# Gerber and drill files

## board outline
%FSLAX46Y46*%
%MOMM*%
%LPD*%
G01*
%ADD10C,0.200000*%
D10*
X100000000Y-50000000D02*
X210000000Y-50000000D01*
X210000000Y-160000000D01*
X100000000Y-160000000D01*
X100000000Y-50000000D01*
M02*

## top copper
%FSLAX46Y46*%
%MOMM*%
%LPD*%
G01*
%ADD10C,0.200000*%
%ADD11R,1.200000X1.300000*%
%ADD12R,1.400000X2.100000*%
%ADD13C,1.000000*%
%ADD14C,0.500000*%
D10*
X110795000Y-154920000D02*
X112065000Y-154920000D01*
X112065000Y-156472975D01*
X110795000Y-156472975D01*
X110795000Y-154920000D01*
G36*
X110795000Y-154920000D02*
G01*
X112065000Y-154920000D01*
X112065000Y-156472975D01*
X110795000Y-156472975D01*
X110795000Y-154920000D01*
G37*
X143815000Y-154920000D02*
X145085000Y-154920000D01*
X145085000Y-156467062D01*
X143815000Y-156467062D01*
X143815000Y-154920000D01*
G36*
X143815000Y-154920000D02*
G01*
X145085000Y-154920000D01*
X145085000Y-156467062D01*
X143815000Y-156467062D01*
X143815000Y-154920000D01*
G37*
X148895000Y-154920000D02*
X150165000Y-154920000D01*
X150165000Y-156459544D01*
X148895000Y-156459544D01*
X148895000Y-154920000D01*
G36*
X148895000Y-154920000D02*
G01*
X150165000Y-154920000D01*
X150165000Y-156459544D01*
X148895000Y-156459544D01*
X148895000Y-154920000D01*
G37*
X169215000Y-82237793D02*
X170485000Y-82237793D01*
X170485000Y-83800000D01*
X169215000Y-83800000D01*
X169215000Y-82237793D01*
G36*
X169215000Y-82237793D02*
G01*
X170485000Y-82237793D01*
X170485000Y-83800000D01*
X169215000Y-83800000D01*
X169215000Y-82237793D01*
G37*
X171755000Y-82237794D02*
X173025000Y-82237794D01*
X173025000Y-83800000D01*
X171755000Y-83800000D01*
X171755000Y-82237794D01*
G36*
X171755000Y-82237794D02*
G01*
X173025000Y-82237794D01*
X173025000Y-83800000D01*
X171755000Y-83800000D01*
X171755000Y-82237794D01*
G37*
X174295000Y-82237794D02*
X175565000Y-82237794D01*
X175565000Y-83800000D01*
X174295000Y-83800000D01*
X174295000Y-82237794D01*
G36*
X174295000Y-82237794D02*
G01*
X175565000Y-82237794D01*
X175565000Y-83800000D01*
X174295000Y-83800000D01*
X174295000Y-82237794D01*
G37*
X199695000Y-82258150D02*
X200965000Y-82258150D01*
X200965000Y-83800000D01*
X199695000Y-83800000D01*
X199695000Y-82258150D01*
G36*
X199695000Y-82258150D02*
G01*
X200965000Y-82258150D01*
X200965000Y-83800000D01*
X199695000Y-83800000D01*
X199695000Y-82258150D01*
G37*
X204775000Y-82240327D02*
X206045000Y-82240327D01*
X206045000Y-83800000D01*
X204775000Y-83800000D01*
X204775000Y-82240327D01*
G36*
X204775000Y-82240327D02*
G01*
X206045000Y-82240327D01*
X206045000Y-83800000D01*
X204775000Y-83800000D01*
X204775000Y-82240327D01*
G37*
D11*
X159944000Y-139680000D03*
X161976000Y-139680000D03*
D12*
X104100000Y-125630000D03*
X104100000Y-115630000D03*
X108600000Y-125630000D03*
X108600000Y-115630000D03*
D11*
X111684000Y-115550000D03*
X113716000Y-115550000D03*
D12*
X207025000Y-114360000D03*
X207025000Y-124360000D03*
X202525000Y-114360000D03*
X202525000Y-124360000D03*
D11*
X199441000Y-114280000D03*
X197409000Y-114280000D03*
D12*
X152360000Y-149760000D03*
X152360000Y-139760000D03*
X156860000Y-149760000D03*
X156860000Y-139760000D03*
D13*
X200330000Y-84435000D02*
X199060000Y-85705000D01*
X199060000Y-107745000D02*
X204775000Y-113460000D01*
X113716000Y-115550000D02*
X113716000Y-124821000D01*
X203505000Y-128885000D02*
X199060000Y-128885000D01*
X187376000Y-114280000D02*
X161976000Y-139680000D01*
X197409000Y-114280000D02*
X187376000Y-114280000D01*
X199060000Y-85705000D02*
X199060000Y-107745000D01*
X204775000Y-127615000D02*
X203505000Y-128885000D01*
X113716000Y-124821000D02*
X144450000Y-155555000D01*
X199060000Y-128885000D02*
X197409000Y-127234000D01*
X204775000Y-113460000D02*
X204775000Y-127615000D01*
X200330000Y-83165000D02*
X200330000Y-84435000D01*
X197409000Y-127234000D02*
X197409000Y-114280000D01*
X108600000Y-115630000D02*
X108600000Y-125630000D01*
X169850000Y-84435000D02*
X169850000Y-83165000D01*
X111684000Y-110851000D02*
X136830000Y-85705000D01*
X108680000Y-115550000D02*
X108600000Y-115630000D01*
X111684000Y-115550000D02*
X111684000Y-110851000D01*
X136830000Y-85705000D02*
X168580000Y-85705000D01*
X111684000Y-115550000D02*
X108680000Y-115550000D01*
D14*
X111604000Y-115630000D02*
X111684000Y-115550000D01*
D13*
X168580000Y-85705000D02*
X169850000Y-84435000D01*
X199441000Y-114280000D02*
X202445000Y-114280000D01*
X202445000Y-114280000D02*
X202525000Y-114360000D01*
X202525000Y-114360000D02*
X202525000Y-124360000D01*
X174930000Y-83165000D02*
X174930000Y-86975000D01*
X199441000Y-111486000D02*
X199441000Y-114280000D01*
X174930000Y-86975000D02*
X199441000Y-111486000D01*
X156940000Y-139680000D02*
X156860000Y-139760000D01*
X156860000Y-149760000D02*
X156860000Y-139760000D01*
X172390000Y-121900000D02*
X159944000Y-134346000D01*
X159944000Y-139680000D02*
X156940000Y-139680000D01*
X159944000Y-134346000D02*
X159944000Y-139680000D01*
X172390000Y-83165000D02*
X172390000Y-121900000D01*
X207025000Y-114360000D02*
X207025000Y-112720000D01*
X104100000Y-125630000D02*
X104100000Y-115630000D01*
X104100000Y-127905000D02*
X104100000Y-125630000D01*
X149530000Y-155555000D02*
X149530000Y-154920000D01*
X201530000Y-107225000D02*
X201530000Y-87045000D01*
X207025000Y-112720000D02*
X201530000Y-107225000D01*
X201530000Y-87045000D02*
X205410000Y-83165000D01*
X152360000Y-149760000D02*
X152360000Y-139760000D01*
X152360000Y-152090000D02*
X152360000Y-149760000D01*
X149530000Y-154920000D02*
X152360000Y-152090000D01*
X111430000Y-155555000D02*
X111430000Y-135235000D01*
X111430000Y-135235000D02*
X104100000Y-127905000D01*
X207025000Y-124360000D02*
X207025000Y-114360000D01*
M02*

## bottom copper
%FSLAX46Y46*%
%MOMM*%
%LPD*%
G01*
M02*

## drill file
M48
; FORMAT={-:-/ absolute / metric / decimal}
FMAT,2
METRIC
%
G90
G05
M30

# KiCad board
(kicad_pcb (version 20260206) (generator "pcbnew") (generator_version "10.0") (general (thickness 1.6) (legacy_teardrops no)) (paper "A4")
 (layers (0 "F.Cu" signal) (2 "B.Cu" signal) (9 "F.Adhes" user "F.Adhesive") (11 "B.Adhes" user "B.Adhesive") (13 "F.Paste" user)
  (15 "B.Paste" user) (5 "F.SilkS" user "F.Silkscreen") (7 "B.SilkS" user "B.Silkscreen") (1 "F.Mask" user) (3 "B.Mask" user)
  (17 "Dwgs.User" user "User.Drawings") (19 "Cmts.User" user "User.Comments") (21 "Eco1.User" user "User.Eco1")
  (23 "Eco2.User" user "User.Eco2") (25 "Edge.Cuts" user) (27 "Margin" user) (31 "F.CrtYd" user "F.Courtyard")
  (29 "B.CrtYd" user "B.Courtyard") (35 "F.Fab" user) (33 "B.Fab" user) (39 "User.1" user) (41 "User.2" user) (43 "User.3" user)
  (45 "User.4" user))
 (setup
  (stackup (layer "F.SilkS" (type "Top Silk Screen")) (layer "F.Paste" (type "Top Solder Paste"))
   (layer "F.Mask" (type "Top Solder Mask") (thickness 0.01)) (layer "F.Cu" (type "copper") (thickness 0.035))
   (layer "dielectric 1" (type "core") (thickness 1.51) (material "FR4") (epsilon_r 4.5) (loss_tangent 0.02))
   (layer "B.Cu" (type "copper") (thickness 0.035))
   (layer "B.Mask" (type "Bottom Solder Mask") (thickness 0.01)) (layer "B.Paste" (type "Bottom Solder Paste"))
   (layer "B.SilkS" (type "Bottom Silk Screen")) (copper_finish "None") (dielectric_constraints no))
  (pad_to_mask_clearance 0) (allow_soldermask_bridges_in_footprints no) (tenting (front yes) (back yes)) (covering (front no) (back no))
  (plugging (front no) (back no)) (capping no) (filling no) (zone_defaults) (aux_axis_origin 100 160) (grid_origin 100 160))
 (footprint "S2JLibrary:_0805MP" (layer "F.Cu") (at 160.96 139.68)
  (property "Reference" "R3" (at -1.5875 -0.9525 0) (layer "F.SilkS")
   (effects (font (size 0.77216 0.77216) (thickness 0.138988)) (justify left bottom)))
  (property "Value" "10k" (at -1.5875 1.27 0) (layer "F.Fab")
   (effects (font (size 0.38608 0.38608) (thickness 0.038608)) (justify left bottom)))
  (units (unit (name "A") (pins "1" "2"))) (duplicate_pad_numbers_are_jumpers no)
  (pad "1" smd rect (at -1.016 0) (size 1.2 1.3) (layers "F.Cu" "F.Mask" "F.Paste") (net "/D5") (solder_mask_margin 0.1016))
  (pad "2" smd rect (at 1.016 0) (size 1.2 1.3) (layers "F.Cu" "F.Mask" "F.Paste") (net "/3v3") (solder_mask_margin 0.1016)))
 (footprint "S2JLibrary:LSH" (layer "F.Cu") (at 106.35 120.63 90)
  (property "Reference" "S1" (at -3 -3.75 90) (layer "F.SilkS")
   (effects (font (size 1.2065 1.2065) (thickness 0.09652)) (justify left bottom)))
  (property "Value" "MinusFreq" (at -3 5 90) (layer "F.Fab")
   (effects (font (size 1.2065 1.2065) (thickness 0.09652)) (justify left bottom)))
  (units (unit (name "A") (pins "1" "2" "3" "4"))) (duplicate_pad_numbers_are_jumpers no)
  (pad "1" smd rect (at -5 -2.25 90) (size 2.1 1.4) (layers "F.Cu" "F.Mask" "F.Paste") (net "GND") (solder_mask_margin 0.1016))
  (pad "2" smd rect (at 5 -2.25 90) (size 2.1 1.4) (layers "F.Cu" "F.Mask" "F.Paste") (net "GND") (solder_mask_margin 0.1016))
  (pad "3" smd rect (at -5 2.25 90) (size 2.1 1.4) (layers "F.Cu" "F.Mask" "F.Paste") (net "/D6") (solder_mask_margin 0.1016))
  (pad "4" smd rect (at 5 2.25 90) (size 2.1 1.4) (layers "F.Cu" "F.Mask" "F.Paste") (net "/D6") (solder_mask_margin 0.1016)))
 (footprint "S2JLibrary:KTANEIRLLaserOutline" (layer "F.Cu") (at 100 160)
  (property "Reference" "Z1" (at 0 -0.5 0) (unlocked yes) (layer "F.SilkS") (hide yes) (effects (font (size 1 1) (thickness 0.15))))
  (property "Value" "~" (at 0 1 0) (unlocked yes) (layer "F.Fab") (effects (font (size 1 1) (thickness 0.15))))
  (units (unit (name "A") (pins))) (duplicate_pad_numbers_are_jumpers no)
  (pad "" smd circle (at 5 -105 180) (size 5.5 5.5) (layers "F.SilkS") (solder_mask_margin 0.1016) (clearance 1))
  (pad "" smd circle (at 5 -55 180) (size 5.5 5.5) (layers "F.SilkS") (solder_mask_margin 0.1016) (clearance 1))
  (pad "" smd circle (at 5 -5 180) (size 5.5 5.5) (layers "F.SilkS") (solder_mask_margin 0.1016) (clearance 1))
  (pad "" smd circle (at 11.43 -2.54 90) (size 1.6764 1.6764) (layers "F.SilkS") (solder_mask_margin 0.1016))
  (pad "" smd circle (at 13.97 -2.54 90) (size 1.6764 1.6764) (layers "F.SilkS") (solder_mask_margin 0.1016))
  (pad "" smd circle (at 16.51 -2.54 90) (size 1.6764 1.6764) (layers "F.SilkS") (solder_mask_margin 0.1016))
  (pad "" smd circle (at 19.05 -2.54 90) (size 1.6764 1.6764) (layers "F.SilkS") (solder_mask_margin 0.1016))
  (pad "" smd circle (at 21.59 -2.54 90) (size 1.6764 1.6764) (layers "F.SilkS") (solder_mask_margin 0.1016))
  (pad "" smd circle (at 24.13 -2.54 90) (size 1.6764 1.6764) (layers "F.SilkS") (solder_mask_margin 0.1016))
  (pad "" smd circle (at 26.67 -2.54 90) (size 1.6764 1.6764) (layers "F.SilkS") (solder_mask_margin 0.1016))
  (pad "" smd circle (at 29.21 -2.54 90) (size 1.6764 1.6764) (layers "F.SilkS") (solder_mask_margin 0.1016))
  (pad "" smd circle (at 31.75 -2.54 90) (size 1.6764 1.6764) (layers "F.SilkS") (solder_mask_margin 0.1016))
  (pad "" smd circle (at 34.29 -2.54 90) (size 1.6764 1.6764) (layers "F.SilkS") (solder_mask_margin 0.1016))
  (pad "" smd circle (at 36.83 -2.54 90) (size 1.6764 1.6764) (layers "F.SilkS") (solder_mask_margin 0.1016))
  (pad "" smd circle (at 39.37 -2.54 90) (size 1.6764 1.6764) (layers "F.SilkS") (solder_mask_margin 0.1016))
  (pad "" smd circle (at 41.91 -2.54 90) (size 1.6764 1.6764) (layers "F.SilkS") (solder_mask_margin 0.1016))
  (pad "" smd circle (at 44.45 -2.54 90) (size 1.6764 1.6764) (layers "F.SilkS") (solder_mask_margin 0.1016))
  (pad "" smd circle (at 46.99 -2.54 90) (size 1.6764 1.6764) (layers "F.SilkS") (solder_mask_margin 0.1016))
  (pad "" smd circle (at 49.53 -2.54 90) (size 1.6764 1.6764) (layers "F.SilkS") (solder_mask_margin 0.1016))
  (pad "" smd circle (at 55 -105 180) (size 5.5 5.5) (layers "F.SilkS") (solder_mask_margin 0.1016) (clearance 1))
  (pad "" smd circle (at 55 -55 180) (size 5.5 5.5) (layers "F.SilkS") (solder_mask_margin 0.1016) (clearance 1))
  (pad "" smd circle (at 55 -5 180) (size 5.5 5.5) (layers "F.SilkS") (solder_mask_margin 0.1016) (clearance 1))
  (pad "" smd circle (at 67.31 -81.28 90) (size 1.6764 1.6764) (layers "F.SilkS") (solder_mask_margin 0.1016))
  (pad "" smd circle (at 67.31 -78.74 90) (size 1.6764 1.6764) (layers "F.SilkS") (solder_mask_margin 0.1016))
  (pad "" smd circle (at 69.85 -81.28 90) (size 1.6764 1.6764) (layers "F.SilkS") (solder_mask_margin 0.1016))
  (pad "" smd circle (at 69.85 -78.74 90) (size 1.6764 1.6764) (layers "F.SilkS") (solder_mask_margin 0.1016))
  (pad "" smd circle (at 72.39 -81.28 90) (size 1.6764 1.6764) (layers "F.SilkS") (solder_mask_margin 0.1016))
  (pad "" smd circle (at 72.39 -78.74 90) (size 1.6764 1.6764) (layers "F.SilkS") (solder_mask_margin 0.1016))
  (pad "" smd circle (at 74.93 -81.28 90) (size 1.6764 1.6764) (layers "F.SilkS") (solder_mask_margin 0.1016))
  (pad "" smd circle (at 74.93 -78.74 90) (size 1.6764 1.6764) (layers "F.SilkS") (solder_mask_margin 0.1016))
  (pad "" smd circle (at 77.47 -81.28 90) (size 1.6764 1.6764) (layers "F.SilkS") (solder_mask_margin 0.1016))
  (pad "" smd circle (at 77.47 -78.74 90) (size 1.6764 1.6764) (layers "F.SilkS") (solder_mask_margin 0.1016))
  (pad "" smd circle (at 80.01 -81.28 90) (size 1.6764 1.6764) (layers "F.SilkS") (solder_mask_margin 0.1016))
  (pad "" smd circle (at 80.01 -78.74 90) (size 1.6764 1.6764) (layers "F.SilkS") (solder_mask_margin 0.1016))
  (pad "" smd circle (at 82.55 -81.28 90) (size 1.6764 1.6764) (layers "F.SilkS") (solder_mask_margin 0.1016))
  (pad "" smd circle (at 82.55 -78.74 90) (size 1.6764 1.6764) (layers "F.SilkS") (solder_mask_margin 0.1016))
  (pad "" smd circle (at 85.09 -81.28 90) (size 1.6764 1.6764) (layers "F.SilkS") (solder_mask_margin 0.1016))
  (pad "" smd circle (at 85.09 -78.74 90) (size 1.6764 1.6764) (layers "F.SilkS") (solder_mask_margin 0.1016))
  (pad "" smd circle (at 87.63 -81.28 90) (size 1.6764 1.6764) (layers "F.SilkS") (solder_mask_margin 0.1016))
  (pad "" smd circle (at 87.63 -78.74 90) (size 1.6764 1.6764) (layers "F.SilkS") (solder_mask_margin 0.1016))
  (pad "" smd circle (at 90.17 -81.28 90) (size 1.6764 1.6764) (layers "F.SilkS") (solder_mask_margin 0.1016))
  (pad "" smd circle (at 90.17 -78.74 90) (size 1.6764 1.6764) (layers "F.SilkS") (solder_mask_margin 0.1016))
  (pad "" smd circle (at 92.71 -81.28 90) (size 1.6764 1.6764) (layers "F.SilkS") (solder_mask_margin 0.1016))
  (pad "" smd circle (at 92.71 -78.74 90) (size 1.6764 1.6764) (layers "F.SilkS") (solder_mask_margin 0.1016))
  (pad "" smd circle (at 95.25 -81.28 90) (size 1.6764 1.6764) (layers "F.SilkS") (solder_mask_margin 0.1016))
  (pad "" smd circle (at 95.25 -78.74 90) (size 1.6764 1.6764) (layers "F.SilkS") (solder_mask_margin 0.1016))
  (pad "" smd circle (at 97.79 -81.28 90) (size 1.6764 1.6764) (layers "F.SilkS") (solder_mask_margin 0.1016))
  (pad "" smd circle (at 97.79 -78.74 90) (size 1.6764 1.6764) (layers "F.SilkS") (solder_mask_margin 0.1016))
  (pad "" smd circle (at 100.33 -81.28 90) (size 1.6764 1.6764) (layers "F.SilkS") (solder_mask_margin 0.1016))
  (pad "" smd circle (at 100.33 -78.74 90) (size 1.6764 1.6764) (layers "F.SilkS") (solder_mask_margin 0.1016))
  (pad "" smd circle (at 102.87 -81.28 90) (size 1.6764 1.6764) (layers "F.SilkS") (solder_mask_margin 0.1016))
  (pad "" smd circle (at 102.87 -78.74 90) (size 1.6764 1.6764) (layers "F.SilkS") (solder_mask_margin 0.1016))
  (pad "" smd circle (at 105 -55 180) (size 5.5 5.5) (layers "F.SilkS") (solder_mask_margin 0.1016) (clearance 1))
  (pad "" smd circle (at 105 -5 180) (size 5.5 5.5) (layers "F.SilkS") (solder_mask_margin 0.1016) (clearance 1))
  (pad "" smd circle (at 105.41 -81.28 90) (size 1.6764 1.6764) (layers "F.SilkS") (solder_mask_margin 0.1016))
  (pad "" smd circle (at 105.41 -78.74 90) (size 1.6764 1.6764) (layers "F.SilkS") (solder_mask_margin 0.1016)))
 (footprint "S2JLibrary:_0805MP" (layer "F.Cu") (at 112.7 115.55)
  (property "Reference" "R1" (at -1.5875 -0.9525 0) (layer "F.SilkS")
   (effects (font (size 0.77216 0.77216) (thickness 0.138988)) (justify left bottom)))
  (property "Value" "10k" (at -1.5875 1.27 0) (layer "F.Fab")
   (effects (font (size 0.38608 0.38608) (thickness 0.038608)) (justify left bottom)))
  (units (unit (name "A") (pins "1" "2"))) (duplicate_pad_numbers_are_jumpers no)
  (pad "1" smd rect (at -1.016 0) (size 1.2 1.3) (layers "F.Cu" "F.Mask" "F.Paste") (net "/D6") (solder_mask_margin 0.1016))
  (pad "2" smd rect (at 1.016 0) (size 1.2 1.3) (layers "F.Cu" "F.Mask" "F.Paste") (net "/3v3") (solder_mask_margin 0.1016)))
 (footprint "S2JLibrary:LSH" (layer "F.Cu") (at 204.775 119.36 -90)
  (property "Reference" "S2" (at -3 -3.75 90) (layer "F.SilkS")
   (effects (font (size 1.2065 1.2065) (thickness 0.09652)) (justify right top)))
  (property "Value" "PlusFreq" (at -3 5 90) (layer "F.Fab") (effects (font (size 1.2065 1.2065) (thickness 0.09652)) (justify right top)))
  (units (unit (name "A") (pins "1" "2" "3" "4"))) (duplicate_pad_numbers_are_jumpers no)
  (pad "1" smd rect (at -5 -2.25 270) (size 2.1 1.4) (layers "F.Cu" "F.Mask" "F.Paste") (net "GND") (solder_mask_margin 0.1016))
  (pad "2" smd rect (at 5 -2.25 270) (size 2.1 1.4) (layers "F.Cu" "F.Mask" "F.Paste") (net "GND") (solder_mask_margin 0.1016))
  (pad "3" smd rect (at -5 2.25 270) (size 2.1 1.4) (layers "F.Cu" "F.Mask" "F.Paste") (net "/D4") (solder_mask_margin 0.1016))
  (pad "4" smd rect (at 5 2.25 270) (size 2.1 1.4) (layers "F.Cu" "F.Mask" "F.Paste") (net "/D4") (solder_mask_margin 0.1016)))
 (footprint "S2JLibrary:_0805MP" (layer "F.Cu") (at 198.425 114.28 180)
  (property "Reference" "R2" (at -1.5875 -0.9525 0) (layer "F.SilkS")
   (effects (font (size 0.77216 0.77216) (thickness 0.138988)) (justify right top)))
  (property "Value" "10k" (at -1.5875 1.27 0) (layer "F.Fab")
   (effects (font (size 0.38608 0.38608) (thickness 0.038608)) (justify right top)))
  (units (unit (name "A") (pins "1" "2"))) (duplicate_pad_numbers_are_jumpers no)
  (pad "1" smd rect (at -1.016 0 180) (size 1.2 1.3) (layers "F.Cu" "F.Mask" "F.Paste") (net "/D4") (solder_mask_margin 0.1016))
  (pad "2" smd rect (at 1.016 0 180) (size 1.2 1.3) (layers "F.Cu" "F.Mask" "F.Paste") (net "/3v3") (solder_mask_margin 0.1016)))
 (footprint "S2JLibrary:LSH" (layer "F.Cu") (at 154.61 144.76 90)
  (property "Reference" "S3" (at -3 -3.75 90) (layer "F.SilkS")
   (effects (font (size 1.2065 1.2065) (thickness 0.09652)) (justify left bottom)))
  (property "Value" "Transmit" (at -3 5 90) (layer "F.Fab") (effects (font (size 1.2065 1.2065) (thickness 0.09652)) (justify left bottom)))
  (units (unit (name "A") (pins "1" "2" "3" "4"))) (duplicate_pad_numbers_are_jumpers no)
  (pad "1" smd rect (at -5 -2.25 90) (size 2.1 1.4) (layers "F.Cu" "F.Mask" "F.Paste") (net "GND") (solder_mask_margin 0.1016))
  (pad "2" smd rect (at 5 -2.25 90) (size 2.1 1.4) (layers "F.Cu" "F.Mask" "F.Paste") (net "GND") (solder_mask_margin 0.1016))
  (pad "3" smd rect (at -5 2.25 90) (size 2.1 1.4) (layers "F.Cu" "F.Mask" "F.Paste") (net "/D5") (solder_mask_margin 0.1016))
  (pad "4" smd rect (at 5 2.25 90) (size 2.1 1.4) (layers "F.Cu" "F.Mask" "F.Paste") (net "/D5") (solder_mask_margin 0.1016)))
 (gr_rect (start 110.795 154.92) (end 112.065 156.472975) (stroke (width 0.2) (type solid)) (fill yes) (layers "F.Cu" "F.Mask") (net "GND"))
 (gr_rect (start 143.815 154.92) (end 145.085 156.467062) (stroke (width 0.2) (type solid)) (fill yes) (layers "F.Cu" "F.Mask") (net "/3v3"))
 (gr_rect (start 148.895 154.92) (end 150.165 156.459544) (stroke (width 0.2) (type solid)) (fill yes) (layers "F.Cu" "F.Mask") (net "GND"))
 (gr_rect (start 169.215 82.237793) (end 170.485 83.8) (stroke (width 0.2) (type solid)) (fill yes) (layers "F.Cu" "F.Mask") (net "/D6"))
 (gr_rect (start 171.755 82.237794) (end 173.025 83.8) (stroke (width 0.2) (type solid)) (fill yes) (layers "F.Cu" "F.Mask") (net "/D5"))
 (gr_rect (start 174.295 82.237794) (end 175.565 83.8) (stroke (width 0.2) (type solid)) (fill yes) (layers "F.Cu" "F.Mask") (net "/D4"))
 (gr_rect (start 199.695 82.25815) (end 200.965 83.8) (stroke (width 0.2) (type solid)) (fill yes) (layers "F.Cu" "F.Mask") (net "/3v3"))
 (gr_rect (start 204.775 82.240327) (end 206.045 83.8) (stroke (width 0.2) (type solid)) (fill yes) (layers "F.Cu" "F.Mask") (net "GND"))
 (gr_rect (start 100 50) (end 210 160) (stroke (width 0.2) (type solid)) (fill no) (layer "Edge.Cuts"))
 (segment (start 200.33 84.435) (end 199.06 85.705) (width 1) (layer "F.Cu") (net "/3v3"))
 (segment (start 199.06 107.745) (end 204.775 113.46) (width 1) (layer "F.Cu") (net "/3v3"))
 (segment (start 113.716 115.55) (end 113.716 124.821) (width 1) (layer "F.Cu") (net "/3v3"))
 (segment (start 203.505 128.885) (end 199.06 128.885) (width 1) (layer "F.Cu") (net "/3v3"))
 (segment (start 187.376 114.28) (end 161.976 139.68) (width 1) (layer "F.Cu") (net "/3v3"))
 (segment (start 197.409 114.28) (end 187.376 114.28) (width 1) (layer "F.Cu") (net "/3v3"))
 (segment (start 199.06 85.705) (end 199.06 107.745) (width 1) (layer "F.Cu") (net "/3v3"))
 (segment (start 204.775 127.615) (end 203.505 128.885) (width 1) (layer "F.Cu") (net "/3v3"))
 (segment (start 113.716 124.821) (end 144.45 155.555) (width 1) (layer "F.Cu") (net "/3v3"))
 (segment (start 199.06 128.885) (end 197.409 127.234) (width 1) (layer "F.Cu") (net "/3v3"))
 (segment (start 204.775 113.46) (end 204.775 127.615) (width 1) (layer "F.Cu") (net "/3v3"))
 (segment (start 200.33 83.165) (end 200.33 84.435) (width 1) (layer "F.Cu") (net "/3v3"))
 (segment (start 197.409 127.234) (end 197.409 114.28) (width 1) (layer "F.Cu") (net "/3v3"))
 (segment (start 108.6 115.63) (end 108.6 125.63) (width 1) (layer "F.Cu") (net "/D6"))
 (segment (start 169.85 84.435) (end 169.85 83.165) (width 1) (layer "F.Cu") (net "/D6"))
 (segment (start 111.684 110.851) (end 136.83 85.705) (width 1) (layer "F.Cu") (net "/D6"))
 (segment (start 108.68 115.55) (end 108.6 115.63) (width 1) (layer "F.Cu") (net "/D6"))
 (segment (start 111.684 115.55) (end 111.684 110.851) (width 1) (layer "F.Cu") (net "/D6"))
 (segment (start 136.83 85.705) (end 168.58 85.705) (width 1) (layer "F.Cu") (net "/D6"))
 (segment (start 111.684 115.55) (end 108.68 115.55) (width 1) (layer "F.Cu") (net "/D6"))
 (segment (start 111.604 115.63) (end 111.684 115.55) (width 0.5) (layer "F.Cu") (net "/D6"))
 (segment (start 168.58 85.705) (end 169.85 84.435) (width 1) (layer "F.Cu") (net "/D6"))
 (segment (start 199.441 114.28) (end 202.445 114.28) (width 1) (layer "F.Cu") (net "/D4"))
 (segment (start 202.445 114.28) (end 202.525 114.36) (width 1) (layer "F.Cu") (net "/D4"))
 (segment (start 202.525 114.36) (end 202.525 124.36) (width 1) (layer "F.Cu") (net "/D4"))
 (segment (start 174.93 83.165) (end 174.93 86.975) (width 1) (layer "F.Cu") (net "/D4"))
 (segment (start 199.441 111.486) (end 199.441 114.28) (width 1) (layer "F.Cu") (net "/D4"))
 (segment (start 174.93 86.975) (end 199.441 111.486) (width 1) (layer "F.Cu") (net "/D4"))
 (segment (start 156.94 139.68) (end 156.86 139.76) (width 1) (layer "F.Cu") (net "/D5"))
 (segment (start 156.86 149.76) (end 156.86 139.76) (width 1) (layer "F.Cu") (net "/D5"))
 (segment (start 172.39 121.9) (end 159.944 134.346) (width 1) (layer "F.Cu") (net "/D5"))
 (segment (start 159.944 139.68) (end 156.94 139.68) (width 1) (layer "F.Cu") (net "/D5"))
 (segment (start 159.944 134.346) (end 159.944 139.68) (width 1) (layer "F.Cu") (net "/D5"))
 (segment (start 172.39 83.165) (end 172.39 121.9) (width 1) (layer "F.Cu") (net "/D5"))
 (segment (start 207.025 114.36) (end 207.025 112.72) (width 1) (layer "F.Cu") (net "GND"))
 (segment (start 104.1 125.63) (end 104.1 115.63) (width 1) (layer "F.Cu") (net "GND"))
 (segment (start 104.1 127.905) (end 104.1 125.63) (width 1) (layer "F.Cu") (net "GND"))
 (segment (start 149.53 155.555) (end 149.53 154.92) (width 1) (layer "F.Cu") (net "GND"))
 (segment (start 201.53 107.225) (end 201.53 87.045) (width 1) (layer "F.Cu") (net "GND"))
 (segment (start 207.025 112.72) (end 201.53 107.225) (width 1) (layer "F.Cu") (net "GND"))
 (segment (start 201.53 87.045) (end 205.41 83.165) (width 1) (layer "F.Cu") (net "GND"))
 (segment (start 152.36 149.76) (end 152.36 139.76) (width 1) (layer "F.Cu") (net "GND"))
 (segment (start 152.36 152.09) (end 152.36 149.76) (width 1) (layer "F.Cu") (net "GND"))
 (segment (start 149.53 154.92) (end 152.36 152.09) (width 1) (layer "F.Cu") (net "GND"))
 (segment (start 111.43 155.555) (end 111.43 135.235) (width 1) (layer "F.Cu") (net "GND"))
 (segment (start 111.43 135.235) (end 104.1 127.905) (width 1) (layer "F.Cu") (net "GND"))
 (segment (start 207.025 124.36) (end 207.025 114.36) (width 1) (layer "F.Cu") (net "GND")))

